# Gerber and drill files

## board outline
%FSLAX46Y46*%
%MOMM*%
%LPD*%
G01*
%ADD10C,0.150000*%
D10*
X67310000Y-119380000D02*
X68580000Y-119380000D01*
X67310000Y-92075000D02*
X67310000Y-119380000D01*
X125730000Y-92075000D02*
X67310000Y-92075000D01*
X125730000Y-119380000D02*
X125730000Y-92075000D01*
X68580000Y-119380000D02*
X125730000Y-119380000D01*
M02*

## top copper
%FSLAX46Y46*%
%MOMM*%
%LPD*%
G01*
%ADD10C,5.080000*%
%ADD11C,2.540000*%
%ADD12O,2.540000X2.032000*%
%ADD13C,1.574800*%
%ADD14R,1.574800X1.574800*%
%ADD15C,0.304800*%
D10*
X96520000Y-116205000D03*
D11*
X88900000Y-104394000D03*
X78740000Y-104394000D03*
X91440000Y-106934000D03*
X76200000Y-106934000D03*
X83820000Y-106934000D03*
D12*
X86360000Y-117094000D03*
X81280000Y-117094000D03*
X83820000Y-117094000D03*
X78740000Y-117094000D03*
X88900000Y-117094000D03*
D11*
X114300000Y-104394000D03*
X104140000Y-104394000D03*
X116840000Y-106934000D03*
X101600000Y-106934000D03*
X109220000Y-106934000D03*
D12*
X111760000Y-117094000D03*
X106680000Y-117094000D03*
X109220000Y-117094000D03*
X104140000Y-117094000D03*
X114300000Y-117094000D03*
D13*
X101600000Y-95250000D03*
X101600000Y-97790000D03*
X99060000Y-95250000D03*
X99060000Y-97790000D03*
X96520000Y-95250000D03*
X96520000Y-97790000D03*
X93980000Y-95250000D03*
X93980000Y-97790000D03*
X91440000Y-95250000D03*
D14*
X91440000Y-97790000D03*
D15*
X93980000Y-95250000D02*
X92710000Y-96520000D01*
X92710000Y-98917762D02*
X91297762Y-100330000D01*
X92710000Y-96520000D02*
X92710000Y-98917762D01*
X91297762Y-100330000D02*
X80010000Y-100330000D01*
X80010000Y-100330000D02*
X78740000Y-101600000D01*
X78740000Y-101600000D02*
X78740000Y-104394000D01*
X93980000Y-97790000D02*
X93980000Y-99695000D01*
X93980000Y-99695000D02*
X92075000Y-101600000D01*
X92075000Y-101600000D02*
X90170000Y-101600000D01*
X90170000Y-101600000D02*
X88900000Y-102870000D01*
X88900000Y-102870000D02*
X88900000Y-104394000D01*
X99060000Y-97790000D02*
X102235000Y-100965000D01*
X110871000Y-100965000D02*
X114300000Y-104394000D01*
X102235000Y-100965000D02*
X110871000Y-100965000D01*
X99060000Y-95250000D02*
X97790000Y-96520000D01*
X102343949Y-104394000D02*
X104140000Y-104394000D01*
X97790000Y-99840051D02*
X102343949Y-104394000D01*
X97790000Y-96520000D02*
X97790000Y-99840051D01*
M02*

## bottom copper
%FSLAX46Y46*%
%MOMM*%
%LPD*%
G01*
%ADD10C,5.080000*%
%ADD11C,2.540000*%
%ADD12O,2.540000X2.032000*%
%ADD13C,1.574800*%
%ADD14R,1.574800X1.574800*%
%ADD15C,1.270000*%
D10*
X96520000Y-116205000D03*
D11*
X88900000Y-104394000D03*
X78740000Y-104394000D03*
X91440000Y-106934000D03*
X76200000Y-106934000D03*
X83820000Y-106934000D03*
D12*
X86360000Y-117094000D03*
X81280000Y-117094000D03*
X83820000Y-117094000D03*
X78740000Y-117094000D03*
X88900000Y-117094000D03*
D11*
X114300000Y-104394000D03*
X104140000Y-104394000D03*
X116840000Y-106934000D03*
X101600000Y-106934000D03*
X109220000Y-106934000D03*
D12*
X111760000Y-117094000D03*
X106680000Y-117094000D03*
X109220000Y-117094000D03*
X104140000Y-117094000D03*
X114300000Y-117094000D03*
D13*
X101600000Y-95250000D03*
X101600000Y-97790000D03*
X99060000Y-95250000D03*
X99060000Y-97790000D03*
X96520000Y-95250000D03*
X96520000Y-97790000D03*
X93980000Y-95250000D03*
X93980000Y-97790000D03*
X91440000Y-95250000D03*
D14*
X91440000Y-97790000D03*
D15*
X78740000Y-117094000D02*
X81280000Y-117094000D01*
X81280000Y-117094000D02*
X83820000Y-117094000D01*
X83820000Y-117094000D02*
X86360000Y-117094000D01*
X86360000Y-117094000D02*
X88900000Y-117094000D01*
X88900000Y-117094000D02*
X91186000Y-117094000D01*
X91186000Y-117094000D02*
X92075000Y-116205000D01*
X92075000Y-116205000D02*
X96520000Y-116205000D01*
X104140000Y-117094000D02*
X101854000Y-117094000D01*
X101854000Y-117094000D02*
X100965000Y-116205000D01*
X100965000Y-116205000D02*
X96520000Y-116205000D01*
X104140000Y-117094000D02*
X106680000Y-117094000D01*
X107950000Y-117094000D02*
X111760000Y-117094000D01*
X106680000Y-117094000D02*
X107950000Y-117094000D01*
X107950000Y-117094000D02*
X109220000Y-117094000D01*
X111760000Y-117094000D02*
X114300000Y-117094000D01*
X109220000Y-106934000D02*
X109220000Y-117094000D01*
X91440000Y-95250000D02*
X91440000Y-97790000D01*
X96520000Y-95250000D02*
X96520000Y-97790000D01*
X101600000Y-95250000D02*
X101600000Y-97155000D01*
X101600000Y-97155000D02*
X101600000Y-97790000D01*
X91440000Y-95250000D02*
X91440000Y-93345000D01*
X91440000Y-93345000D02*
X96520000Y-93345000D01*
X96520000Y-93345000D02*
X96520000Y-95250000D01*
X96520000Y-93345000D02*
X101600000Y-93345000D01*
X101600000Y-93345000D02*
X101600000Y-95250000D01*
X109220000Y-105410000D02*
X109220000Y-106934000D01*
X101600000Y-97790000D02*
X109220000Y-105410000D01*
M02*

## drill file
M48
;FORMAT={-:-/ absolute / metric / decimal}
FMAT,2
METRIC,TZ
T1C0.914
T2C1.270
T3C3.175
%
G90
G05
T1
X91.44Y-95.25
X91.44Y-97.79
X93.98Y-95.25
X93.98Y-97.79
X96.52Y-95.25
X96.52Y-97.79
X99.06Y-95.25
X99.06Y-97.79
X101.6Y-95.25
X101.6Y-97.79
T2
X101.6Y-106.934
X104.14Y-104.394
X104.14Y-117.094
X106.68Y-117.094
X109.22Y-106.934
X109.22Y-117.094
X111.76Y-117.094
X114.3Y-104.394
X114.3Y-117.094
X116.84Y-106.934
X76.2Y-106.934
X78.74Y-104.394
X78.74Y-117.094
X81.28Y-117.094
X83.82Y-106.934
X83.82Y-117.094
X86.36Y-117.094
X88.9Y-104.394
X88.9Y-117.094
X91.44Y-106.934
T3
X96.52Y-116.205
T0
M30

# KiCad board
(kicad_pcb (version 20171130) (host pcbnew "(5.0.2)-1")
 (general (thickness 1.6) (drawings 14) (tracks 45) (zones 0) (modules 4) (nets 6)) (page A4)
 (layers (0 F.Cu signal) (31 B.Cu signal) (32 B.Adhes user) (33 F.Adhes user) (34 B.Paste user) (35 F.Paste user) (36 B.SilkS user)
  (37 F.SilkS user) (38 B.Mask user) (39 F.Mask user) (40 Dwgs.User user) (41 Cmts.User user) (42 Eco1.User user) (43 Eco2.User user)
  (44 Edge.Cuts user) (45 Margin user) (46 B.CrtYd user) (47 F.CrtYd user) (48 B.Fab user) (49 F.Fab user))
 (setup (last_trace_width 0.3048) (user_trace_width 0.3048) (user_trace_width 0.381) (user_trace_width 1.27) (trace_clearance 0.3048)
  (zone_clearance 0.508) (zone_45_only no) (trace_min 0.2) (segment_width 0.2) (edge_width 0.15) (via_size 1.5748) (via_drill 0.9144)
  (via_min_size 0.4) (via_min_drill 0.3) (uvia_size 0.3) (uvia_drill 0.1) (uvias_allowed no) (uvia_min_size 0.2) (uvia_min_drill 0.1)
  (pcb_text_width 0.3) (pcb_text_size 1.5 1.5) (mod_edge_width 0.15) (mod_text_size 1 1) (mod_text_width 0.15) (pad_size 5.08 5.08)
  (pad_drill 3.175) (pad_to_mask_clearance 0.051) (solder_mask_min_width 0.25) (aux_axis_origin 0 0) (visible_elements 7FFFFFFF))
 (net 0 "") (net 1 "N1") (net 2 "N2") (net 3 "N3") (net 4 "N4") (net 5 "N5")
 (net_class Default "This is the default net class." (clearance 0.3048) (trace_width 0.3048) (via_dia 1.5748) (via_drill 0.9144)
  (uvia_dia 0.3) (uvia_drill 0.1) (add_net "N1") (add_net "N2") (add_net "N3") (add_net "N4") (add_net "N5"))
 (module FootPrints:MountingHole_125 (layer F.Cu) (at 96.52 116.205)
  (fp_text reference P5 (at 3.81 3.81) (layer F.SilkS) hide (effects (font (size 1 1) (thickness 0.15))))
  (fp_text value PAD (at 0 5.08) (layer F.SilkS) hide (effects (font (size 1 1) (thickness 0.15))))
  (pad 1 thru_hole circle (at 0 0) (size 5.08 5.08) (drill 3.175) (layers *.Cu *.Mask F.SilkS) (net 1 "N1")))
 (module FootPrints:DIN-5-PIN (layer F.Cu) (at 83.82 119.38)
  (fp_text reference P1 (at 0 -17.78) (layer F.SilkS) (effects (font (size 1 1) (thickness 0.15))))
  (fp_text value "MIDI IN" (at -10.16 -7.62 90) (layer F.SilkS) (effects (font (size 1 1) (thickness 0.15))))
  (pad 4 thru_hole circle (at 5.08 -14.986) (size 2.54 2.54) (drill 1.27) (layers *.Cu *.Mask F.SilkS) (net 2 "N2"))
  (pad 5 thru_hole circle (at -5.08 -14.986) (size 2.54 2.54) (drill 1.27) (layers *.Cu *.Mask F.SilkS) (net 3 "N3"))
  (pad 1 thru_hole circle (at 7.62 -12.446) (size 2.54 2.54) (drill 1.27) (layers *.Cu *.Mask F.SilkS))
  (pad 3 thru_hole circle (at -7.62 -12.446) (size 2.54 2.54) (drill 1.27) (layers *.Cu *.Mask F.SilkS))
  (pad 2 thru_hole circle (at 0 -12.446) (size 2.54 2.54) (drill 1.27) (layers *.Cu *.Mask F.SilkS))
  (pad 7 thru_hole oval (at 2.54 -2.286) (size 2.54 2.032) (drill 1.27) (layers *.Cu *.Mask F.SilkS) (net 1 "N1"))
  (pad 6 thru_hole oval (at -2.54 -2.286) (size 2.54 2.032) (drill 1.27) (layers *.Cu *.Mask F.SilkS) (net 1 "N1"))
  (pad 9 thru_hole oval (at 0 -2.286) (size 2.54 2.032) (drill 1.27) (layers *.Cu *.Mask F.SilkS) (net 1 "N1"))
  (pad 8 thru_hole oval (at -5.08 -2.286) (size 2.54 2.032) (drill 1.27) (layers *.Cu *.Mask F.SilkS) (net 1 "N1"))
  (pad 10 thru_hole oval (at 5.08 -2.286) (size 2.54 2.032) (drill 1.27) (layers *.Cu *.Mask F.SilkS) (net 1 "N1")))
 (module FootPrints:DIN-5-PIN (layer F.Cu) (at 109.22 119.38)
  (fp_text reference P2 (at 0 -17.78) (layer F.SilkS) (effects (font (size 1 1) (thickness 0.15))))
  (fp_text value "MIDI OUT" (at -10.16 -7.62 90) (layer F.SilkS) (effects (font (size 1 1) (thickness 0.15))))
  (pad 4 thru_hole circle (at 5.08 -14.986) (size 2.54 2.54) (drill 1.27) (layers *.Cu *.Mask F.SilkS) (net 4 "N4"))
  (pad 5 thru_hole circle (at -5.08 -14.986) (size 2.54 2.54) (drill 1.27) (layers *.Cu *.Mask F.SilkS) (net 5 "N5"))
  (pad 1 thru_hole circle (at 7.62 -12.446) (size 2.54 2.54) (drill 1.27) (layers *.Cu *.Mask F.SilkS))
  (pad 3 thru_hole circle (at -7.62 -12.446) (size 2.54 2.54) (drill 1.27) (layers *.Cu *.Mask F.SilkS))
  (pad 2 thru_hole circle (at 0 -12.446) (size 2.54 2.54) (drill 1.27) (layers *.Cu *.Mask F.SilkS) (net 1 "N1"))
  (pad 7 thru_hole oval (at 2.54 -2.286) (size 2.54 2.032) (drill 1.27) (layers *.Cu *.Mask F.SilkS) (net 1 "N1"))
  (pad 6 thru_hole oval (at -2.54 -2.286) (size 2.54 2.032) (drill 1.27) (layers *.Cu *.Mask F.SilkS) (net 1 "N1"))
  (pad 9 thru_hole oval (at 0 -2.286) (size 2.54 2.032) (drill 1.27) (layers *.Cu *.Mask F.SilkS) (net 1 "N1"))
  (pad 8 thru_hole oval (at -5.08 -2.286) (size 2.54 2.032) (drill 1.27) (layers *.Cu *.Mask F.SilkS) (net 1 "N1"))
  (pad 10 thru_hole oval (at 5.08 -2.286) (size 2.54 2.032) (drill 1.27) (layers *.Cu *.Mask F.SilkS) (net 1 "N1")))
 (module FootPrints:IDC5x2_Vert (layer F.Cu) (at 96.52 96.52 180)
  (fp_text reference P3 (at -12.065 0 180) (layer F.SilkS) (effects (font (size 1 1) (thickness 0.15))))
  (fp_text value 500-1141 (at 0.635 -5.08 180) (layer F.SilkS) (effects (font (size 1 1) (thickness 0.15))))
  (pad 10 thru_hole circle (at -5.08 1.27 180) (size 1.5748 1.5748) (drill 0.9144) (layers *.Cu *.Mask F.SilkS) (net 1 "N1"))
  (pad 9 thru_hole circle (at -5.08 -1.27 180) (size 1.5748 1.5748) (drill 0.9144) (layers *.Cu *.Mask F.SilkS) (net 1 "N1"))
  (pad 8 thru_hole circle (at -2.54 1.27 180) (size 1.5748 1.5748) (drill 0.9144) (layers *.Cu *.Mask F.SilkS) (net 5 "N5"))
  (pad 7 thru_hole circle (at -2.54 -1.27 180) (size 1.5748 1.5748) (drill 0.9144) (layers *.Cu *.Mask F.SilkS) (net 4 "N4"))
  (pad 6 thru_hole circle (at 0 1.27 180) (size 1.5748 1.5748) (drill 0.9144) (layers *.Cu *.Mask F.SilkS) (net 1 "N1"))
  (pad 5 thru_hole circle (at 0 -1.27 180) (size 1.5748 1.5748) (drill 0.9144) (layers *.Cu *.Mask F.SilkS) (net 1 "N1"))
  (pad 4 thru_hole circle (at 2.54 1.27 180) (size 1.5748 1.5748) (drill 0.9144) (layers *.Cu *.Mask F.SilkS) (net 3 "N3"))
  (pad 3 thru_hole circle (at 2.54 -1.27 180) (size 1.5748 1.5748) (drill 0.9144) (layers *.Cu *.Mask F.SilkS) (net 2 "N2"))
  (pad 2 thru_hole circle (at 5.08 1.27 180) (size 1.5748 1.5748) (drill 0.9144) (layers *.Cu *.Mask F.SilkS) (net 1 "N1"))
  (pad 1 thru_hole rect (at 5.08 -1.27 180) (size 1.5748 1.5748) (drill 0.9144) (layers *.Cu *.Mask F.SilkS) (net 1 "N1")))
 (gr_line (start 67.31 119.38) (end 68.58 119.38) (layer Edge.Cuts) (width 0.15))
 (gr_line (start 67.31 92.075) (end 67.31 119.38) (layer Edge.Cuts) (width 0.15))
 (gr_line (start 125.73 92.075) (end 67.31 92.075) (layer Edge.Cuts) (width 0.15))
 (gr_line (start 125.73 119.38) (end 125.73 92.075) (layer Edge.Cuts) (width 0.15))
 (gr_line (start 68.58 119.38) (end 125.73 119.38) (layer Edge.Cuts) (width 0.15))
 (segment (start 78.74 117.094) (end 81.28 117.094) (width 1.27) (layer B.Cu) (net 1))
 (segment (start 81.28 117.094) (end 83.82 117.094) (width 1.27) (layer B.Cu) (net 1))
 (segment (start 83.82 117.094) (end 86.36 117.094) (width 1.27) (layer B.Cu) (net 1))
 (segment (start 86.36 117.094) (end 88.9 117.094) (width 1.27) (layer B.Cu) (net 1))
 (segment (start 88.9 117.094) (end 91.186 117.094) (width 1.27) (layer B.Cu) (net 1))
 (segment (start 91.186 117.094) (end 92.075 116.205) (width 1.27) (layer B.Cu) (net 1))
 (segment (start 92.075 116.205) (end 96.52 116.205) (width 1.27) (layer B.Cu) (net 1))
 (segment (start 104.14 117.094) (end 101.854 117.094) (width 1.27) (layer B.Cu) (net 1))
 (segment (start 101.854 117.094) (end 100.965 116.205) (width 1.27) (layer B.Cu) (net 1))
 (segment (start 100.965 116.205) (end 96.52 116.205) (width 1.27) (layer B.Cu) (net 1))
 (segment (start 104.14 117.094) (end 106.68 117.094) (width 1.27) (layer B.Cu) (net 1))
 (segment (start 107.95 117.094) (end 111.76 117.094) (width 1.27) (layer B.Cu) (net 1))
 (segment (start 106.68 117.094) (end 107.95 117.094) (width 1.27) (layer B.Cu) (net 1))
 (segment (start 107.95 117.094) (end 109.22 117.094) (width 1.27) (layer B.Cu) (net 1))
 (segment (start 111.76 117.094) (end 114.3 117.094) (width 1.27) (layer B.Cu) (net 1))
 (segment (start 109.22 106.934) (end 109.22 117.094) (width 1.27) (layer B.Cu) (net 1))
 (segment (start 91.44 95.25) (end 91.44 97.79) (width 1.27) (layer B.Cu) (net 1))
 (segment (start 96.52 95.25) (end 96.52 97.79) (width 1.27) (layer B.Cu) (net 1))
 (segment (start 101.6 95.25) (end 101.6 97.155) (width 1.27) (layer B.Cu) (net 1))
 (segment (start 101.6 97.155) (end 101.6 97.79) (width 1.27) (layer B.Cu) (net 1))
 (segment (start 91.44 95.25) (end 91.44 93.345) (width 1.27) (layer B.Cu) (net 1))
 (segment (start 91.44 93.345) (end 96.52 93.345) (width 1.27) (layer B.Cu) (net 1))
 (segment (start 96.52 93.345) (end 96.52 95.25) (width 1.27) (layer B.Cu) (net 1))
 (segment (start 96.52 93.345) (end 101.6 93.345) (width 1.27) (layer B.Cu) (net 1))
 (segment (start 101.6 93.345) (end 101.6 95.25) (width 1.27) (layer B.Cu) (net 1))
 (segment (start 109.22 105.41) (end 109.22 106.934) (width 1.27) (layer B.Cu) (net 1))
 (segment (start 101.6 97.79) (end 109.22 105.41) (width 1.27) (layer B.Cu) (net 1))
 (segment (start 93.98 95.25) (end 92.71 96.52) (width 0.3048) (layer F.Cu) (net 3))
 (segment (start 92.71 98.917762) (end 91.297762 100.33) (width 0.3048) (layer F.Cu) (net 3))
 (segment (start 92.71 96.52) (end 92.71 98.917762) (width 0.3048) (layer F.Cu) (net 3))
 (segment (start 91.297762 100.33) (end 80.01 100.33) (width 0.3048) (layer F.Cu) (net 3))
 (segment (start 80.01 100.33) (end 78.74 101.6) (width 0.3048) (layer F.Cu) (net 3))
 (segment (start 78.74 101.6) (end 78.74 104.394) (width 0.3048) (layer F.Cu) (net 3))
 (segment (start 93.98 97.79) (end 93.98 99.695) (width 0.3048) (layer F.Cu) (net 2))
 (segment (start 93.98 99.695) (end 92.075 101.6) (width 0.3048) (layer F.Cu) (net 2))
 (segment (start 92.075 101.6) (end 90.17 101.6) (width 0.3048) (layer F.Cu) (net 2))
 (segment (start 90.17 101.6) (end 88.9 102.87) (width 0.3048) (layer F.Cu) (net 2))
 (segment (start 88.9 102.87) (end 88.9 104.394) (width 0.3048) (layer F.Cu) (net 2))
 (segment (start 99.06 97.79) (end 102.235 100.965) (width 0.3048) (layer F.Cu) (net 4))
 (segment (start 110.871 100.965) (end 114.3 104.394) (width 0.3048) (layer F.Cu) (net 4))
 (segment (start 102.235 100.965) (end 110.871 100.965) (width 0.3048) (layer F.Cu) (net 4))
 (segment (start 99.06 95.25) (end 97.79 96.52) (width 0.3048) (layer F.Cu) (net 5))
 (segment (start 102.343949 104.394) (end 104.14 104.394) (width 0.3048) (layer F.Cu) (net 5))
 (segment (start 97.79 99.840051) (end 102.343949 104.394) (width 0.3048) (layer F.Cu) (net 5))
 (segment (start 97.79 96.52) (end 97.79 99.840051) (width 0.3048) (layer F.Cu) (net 5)))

